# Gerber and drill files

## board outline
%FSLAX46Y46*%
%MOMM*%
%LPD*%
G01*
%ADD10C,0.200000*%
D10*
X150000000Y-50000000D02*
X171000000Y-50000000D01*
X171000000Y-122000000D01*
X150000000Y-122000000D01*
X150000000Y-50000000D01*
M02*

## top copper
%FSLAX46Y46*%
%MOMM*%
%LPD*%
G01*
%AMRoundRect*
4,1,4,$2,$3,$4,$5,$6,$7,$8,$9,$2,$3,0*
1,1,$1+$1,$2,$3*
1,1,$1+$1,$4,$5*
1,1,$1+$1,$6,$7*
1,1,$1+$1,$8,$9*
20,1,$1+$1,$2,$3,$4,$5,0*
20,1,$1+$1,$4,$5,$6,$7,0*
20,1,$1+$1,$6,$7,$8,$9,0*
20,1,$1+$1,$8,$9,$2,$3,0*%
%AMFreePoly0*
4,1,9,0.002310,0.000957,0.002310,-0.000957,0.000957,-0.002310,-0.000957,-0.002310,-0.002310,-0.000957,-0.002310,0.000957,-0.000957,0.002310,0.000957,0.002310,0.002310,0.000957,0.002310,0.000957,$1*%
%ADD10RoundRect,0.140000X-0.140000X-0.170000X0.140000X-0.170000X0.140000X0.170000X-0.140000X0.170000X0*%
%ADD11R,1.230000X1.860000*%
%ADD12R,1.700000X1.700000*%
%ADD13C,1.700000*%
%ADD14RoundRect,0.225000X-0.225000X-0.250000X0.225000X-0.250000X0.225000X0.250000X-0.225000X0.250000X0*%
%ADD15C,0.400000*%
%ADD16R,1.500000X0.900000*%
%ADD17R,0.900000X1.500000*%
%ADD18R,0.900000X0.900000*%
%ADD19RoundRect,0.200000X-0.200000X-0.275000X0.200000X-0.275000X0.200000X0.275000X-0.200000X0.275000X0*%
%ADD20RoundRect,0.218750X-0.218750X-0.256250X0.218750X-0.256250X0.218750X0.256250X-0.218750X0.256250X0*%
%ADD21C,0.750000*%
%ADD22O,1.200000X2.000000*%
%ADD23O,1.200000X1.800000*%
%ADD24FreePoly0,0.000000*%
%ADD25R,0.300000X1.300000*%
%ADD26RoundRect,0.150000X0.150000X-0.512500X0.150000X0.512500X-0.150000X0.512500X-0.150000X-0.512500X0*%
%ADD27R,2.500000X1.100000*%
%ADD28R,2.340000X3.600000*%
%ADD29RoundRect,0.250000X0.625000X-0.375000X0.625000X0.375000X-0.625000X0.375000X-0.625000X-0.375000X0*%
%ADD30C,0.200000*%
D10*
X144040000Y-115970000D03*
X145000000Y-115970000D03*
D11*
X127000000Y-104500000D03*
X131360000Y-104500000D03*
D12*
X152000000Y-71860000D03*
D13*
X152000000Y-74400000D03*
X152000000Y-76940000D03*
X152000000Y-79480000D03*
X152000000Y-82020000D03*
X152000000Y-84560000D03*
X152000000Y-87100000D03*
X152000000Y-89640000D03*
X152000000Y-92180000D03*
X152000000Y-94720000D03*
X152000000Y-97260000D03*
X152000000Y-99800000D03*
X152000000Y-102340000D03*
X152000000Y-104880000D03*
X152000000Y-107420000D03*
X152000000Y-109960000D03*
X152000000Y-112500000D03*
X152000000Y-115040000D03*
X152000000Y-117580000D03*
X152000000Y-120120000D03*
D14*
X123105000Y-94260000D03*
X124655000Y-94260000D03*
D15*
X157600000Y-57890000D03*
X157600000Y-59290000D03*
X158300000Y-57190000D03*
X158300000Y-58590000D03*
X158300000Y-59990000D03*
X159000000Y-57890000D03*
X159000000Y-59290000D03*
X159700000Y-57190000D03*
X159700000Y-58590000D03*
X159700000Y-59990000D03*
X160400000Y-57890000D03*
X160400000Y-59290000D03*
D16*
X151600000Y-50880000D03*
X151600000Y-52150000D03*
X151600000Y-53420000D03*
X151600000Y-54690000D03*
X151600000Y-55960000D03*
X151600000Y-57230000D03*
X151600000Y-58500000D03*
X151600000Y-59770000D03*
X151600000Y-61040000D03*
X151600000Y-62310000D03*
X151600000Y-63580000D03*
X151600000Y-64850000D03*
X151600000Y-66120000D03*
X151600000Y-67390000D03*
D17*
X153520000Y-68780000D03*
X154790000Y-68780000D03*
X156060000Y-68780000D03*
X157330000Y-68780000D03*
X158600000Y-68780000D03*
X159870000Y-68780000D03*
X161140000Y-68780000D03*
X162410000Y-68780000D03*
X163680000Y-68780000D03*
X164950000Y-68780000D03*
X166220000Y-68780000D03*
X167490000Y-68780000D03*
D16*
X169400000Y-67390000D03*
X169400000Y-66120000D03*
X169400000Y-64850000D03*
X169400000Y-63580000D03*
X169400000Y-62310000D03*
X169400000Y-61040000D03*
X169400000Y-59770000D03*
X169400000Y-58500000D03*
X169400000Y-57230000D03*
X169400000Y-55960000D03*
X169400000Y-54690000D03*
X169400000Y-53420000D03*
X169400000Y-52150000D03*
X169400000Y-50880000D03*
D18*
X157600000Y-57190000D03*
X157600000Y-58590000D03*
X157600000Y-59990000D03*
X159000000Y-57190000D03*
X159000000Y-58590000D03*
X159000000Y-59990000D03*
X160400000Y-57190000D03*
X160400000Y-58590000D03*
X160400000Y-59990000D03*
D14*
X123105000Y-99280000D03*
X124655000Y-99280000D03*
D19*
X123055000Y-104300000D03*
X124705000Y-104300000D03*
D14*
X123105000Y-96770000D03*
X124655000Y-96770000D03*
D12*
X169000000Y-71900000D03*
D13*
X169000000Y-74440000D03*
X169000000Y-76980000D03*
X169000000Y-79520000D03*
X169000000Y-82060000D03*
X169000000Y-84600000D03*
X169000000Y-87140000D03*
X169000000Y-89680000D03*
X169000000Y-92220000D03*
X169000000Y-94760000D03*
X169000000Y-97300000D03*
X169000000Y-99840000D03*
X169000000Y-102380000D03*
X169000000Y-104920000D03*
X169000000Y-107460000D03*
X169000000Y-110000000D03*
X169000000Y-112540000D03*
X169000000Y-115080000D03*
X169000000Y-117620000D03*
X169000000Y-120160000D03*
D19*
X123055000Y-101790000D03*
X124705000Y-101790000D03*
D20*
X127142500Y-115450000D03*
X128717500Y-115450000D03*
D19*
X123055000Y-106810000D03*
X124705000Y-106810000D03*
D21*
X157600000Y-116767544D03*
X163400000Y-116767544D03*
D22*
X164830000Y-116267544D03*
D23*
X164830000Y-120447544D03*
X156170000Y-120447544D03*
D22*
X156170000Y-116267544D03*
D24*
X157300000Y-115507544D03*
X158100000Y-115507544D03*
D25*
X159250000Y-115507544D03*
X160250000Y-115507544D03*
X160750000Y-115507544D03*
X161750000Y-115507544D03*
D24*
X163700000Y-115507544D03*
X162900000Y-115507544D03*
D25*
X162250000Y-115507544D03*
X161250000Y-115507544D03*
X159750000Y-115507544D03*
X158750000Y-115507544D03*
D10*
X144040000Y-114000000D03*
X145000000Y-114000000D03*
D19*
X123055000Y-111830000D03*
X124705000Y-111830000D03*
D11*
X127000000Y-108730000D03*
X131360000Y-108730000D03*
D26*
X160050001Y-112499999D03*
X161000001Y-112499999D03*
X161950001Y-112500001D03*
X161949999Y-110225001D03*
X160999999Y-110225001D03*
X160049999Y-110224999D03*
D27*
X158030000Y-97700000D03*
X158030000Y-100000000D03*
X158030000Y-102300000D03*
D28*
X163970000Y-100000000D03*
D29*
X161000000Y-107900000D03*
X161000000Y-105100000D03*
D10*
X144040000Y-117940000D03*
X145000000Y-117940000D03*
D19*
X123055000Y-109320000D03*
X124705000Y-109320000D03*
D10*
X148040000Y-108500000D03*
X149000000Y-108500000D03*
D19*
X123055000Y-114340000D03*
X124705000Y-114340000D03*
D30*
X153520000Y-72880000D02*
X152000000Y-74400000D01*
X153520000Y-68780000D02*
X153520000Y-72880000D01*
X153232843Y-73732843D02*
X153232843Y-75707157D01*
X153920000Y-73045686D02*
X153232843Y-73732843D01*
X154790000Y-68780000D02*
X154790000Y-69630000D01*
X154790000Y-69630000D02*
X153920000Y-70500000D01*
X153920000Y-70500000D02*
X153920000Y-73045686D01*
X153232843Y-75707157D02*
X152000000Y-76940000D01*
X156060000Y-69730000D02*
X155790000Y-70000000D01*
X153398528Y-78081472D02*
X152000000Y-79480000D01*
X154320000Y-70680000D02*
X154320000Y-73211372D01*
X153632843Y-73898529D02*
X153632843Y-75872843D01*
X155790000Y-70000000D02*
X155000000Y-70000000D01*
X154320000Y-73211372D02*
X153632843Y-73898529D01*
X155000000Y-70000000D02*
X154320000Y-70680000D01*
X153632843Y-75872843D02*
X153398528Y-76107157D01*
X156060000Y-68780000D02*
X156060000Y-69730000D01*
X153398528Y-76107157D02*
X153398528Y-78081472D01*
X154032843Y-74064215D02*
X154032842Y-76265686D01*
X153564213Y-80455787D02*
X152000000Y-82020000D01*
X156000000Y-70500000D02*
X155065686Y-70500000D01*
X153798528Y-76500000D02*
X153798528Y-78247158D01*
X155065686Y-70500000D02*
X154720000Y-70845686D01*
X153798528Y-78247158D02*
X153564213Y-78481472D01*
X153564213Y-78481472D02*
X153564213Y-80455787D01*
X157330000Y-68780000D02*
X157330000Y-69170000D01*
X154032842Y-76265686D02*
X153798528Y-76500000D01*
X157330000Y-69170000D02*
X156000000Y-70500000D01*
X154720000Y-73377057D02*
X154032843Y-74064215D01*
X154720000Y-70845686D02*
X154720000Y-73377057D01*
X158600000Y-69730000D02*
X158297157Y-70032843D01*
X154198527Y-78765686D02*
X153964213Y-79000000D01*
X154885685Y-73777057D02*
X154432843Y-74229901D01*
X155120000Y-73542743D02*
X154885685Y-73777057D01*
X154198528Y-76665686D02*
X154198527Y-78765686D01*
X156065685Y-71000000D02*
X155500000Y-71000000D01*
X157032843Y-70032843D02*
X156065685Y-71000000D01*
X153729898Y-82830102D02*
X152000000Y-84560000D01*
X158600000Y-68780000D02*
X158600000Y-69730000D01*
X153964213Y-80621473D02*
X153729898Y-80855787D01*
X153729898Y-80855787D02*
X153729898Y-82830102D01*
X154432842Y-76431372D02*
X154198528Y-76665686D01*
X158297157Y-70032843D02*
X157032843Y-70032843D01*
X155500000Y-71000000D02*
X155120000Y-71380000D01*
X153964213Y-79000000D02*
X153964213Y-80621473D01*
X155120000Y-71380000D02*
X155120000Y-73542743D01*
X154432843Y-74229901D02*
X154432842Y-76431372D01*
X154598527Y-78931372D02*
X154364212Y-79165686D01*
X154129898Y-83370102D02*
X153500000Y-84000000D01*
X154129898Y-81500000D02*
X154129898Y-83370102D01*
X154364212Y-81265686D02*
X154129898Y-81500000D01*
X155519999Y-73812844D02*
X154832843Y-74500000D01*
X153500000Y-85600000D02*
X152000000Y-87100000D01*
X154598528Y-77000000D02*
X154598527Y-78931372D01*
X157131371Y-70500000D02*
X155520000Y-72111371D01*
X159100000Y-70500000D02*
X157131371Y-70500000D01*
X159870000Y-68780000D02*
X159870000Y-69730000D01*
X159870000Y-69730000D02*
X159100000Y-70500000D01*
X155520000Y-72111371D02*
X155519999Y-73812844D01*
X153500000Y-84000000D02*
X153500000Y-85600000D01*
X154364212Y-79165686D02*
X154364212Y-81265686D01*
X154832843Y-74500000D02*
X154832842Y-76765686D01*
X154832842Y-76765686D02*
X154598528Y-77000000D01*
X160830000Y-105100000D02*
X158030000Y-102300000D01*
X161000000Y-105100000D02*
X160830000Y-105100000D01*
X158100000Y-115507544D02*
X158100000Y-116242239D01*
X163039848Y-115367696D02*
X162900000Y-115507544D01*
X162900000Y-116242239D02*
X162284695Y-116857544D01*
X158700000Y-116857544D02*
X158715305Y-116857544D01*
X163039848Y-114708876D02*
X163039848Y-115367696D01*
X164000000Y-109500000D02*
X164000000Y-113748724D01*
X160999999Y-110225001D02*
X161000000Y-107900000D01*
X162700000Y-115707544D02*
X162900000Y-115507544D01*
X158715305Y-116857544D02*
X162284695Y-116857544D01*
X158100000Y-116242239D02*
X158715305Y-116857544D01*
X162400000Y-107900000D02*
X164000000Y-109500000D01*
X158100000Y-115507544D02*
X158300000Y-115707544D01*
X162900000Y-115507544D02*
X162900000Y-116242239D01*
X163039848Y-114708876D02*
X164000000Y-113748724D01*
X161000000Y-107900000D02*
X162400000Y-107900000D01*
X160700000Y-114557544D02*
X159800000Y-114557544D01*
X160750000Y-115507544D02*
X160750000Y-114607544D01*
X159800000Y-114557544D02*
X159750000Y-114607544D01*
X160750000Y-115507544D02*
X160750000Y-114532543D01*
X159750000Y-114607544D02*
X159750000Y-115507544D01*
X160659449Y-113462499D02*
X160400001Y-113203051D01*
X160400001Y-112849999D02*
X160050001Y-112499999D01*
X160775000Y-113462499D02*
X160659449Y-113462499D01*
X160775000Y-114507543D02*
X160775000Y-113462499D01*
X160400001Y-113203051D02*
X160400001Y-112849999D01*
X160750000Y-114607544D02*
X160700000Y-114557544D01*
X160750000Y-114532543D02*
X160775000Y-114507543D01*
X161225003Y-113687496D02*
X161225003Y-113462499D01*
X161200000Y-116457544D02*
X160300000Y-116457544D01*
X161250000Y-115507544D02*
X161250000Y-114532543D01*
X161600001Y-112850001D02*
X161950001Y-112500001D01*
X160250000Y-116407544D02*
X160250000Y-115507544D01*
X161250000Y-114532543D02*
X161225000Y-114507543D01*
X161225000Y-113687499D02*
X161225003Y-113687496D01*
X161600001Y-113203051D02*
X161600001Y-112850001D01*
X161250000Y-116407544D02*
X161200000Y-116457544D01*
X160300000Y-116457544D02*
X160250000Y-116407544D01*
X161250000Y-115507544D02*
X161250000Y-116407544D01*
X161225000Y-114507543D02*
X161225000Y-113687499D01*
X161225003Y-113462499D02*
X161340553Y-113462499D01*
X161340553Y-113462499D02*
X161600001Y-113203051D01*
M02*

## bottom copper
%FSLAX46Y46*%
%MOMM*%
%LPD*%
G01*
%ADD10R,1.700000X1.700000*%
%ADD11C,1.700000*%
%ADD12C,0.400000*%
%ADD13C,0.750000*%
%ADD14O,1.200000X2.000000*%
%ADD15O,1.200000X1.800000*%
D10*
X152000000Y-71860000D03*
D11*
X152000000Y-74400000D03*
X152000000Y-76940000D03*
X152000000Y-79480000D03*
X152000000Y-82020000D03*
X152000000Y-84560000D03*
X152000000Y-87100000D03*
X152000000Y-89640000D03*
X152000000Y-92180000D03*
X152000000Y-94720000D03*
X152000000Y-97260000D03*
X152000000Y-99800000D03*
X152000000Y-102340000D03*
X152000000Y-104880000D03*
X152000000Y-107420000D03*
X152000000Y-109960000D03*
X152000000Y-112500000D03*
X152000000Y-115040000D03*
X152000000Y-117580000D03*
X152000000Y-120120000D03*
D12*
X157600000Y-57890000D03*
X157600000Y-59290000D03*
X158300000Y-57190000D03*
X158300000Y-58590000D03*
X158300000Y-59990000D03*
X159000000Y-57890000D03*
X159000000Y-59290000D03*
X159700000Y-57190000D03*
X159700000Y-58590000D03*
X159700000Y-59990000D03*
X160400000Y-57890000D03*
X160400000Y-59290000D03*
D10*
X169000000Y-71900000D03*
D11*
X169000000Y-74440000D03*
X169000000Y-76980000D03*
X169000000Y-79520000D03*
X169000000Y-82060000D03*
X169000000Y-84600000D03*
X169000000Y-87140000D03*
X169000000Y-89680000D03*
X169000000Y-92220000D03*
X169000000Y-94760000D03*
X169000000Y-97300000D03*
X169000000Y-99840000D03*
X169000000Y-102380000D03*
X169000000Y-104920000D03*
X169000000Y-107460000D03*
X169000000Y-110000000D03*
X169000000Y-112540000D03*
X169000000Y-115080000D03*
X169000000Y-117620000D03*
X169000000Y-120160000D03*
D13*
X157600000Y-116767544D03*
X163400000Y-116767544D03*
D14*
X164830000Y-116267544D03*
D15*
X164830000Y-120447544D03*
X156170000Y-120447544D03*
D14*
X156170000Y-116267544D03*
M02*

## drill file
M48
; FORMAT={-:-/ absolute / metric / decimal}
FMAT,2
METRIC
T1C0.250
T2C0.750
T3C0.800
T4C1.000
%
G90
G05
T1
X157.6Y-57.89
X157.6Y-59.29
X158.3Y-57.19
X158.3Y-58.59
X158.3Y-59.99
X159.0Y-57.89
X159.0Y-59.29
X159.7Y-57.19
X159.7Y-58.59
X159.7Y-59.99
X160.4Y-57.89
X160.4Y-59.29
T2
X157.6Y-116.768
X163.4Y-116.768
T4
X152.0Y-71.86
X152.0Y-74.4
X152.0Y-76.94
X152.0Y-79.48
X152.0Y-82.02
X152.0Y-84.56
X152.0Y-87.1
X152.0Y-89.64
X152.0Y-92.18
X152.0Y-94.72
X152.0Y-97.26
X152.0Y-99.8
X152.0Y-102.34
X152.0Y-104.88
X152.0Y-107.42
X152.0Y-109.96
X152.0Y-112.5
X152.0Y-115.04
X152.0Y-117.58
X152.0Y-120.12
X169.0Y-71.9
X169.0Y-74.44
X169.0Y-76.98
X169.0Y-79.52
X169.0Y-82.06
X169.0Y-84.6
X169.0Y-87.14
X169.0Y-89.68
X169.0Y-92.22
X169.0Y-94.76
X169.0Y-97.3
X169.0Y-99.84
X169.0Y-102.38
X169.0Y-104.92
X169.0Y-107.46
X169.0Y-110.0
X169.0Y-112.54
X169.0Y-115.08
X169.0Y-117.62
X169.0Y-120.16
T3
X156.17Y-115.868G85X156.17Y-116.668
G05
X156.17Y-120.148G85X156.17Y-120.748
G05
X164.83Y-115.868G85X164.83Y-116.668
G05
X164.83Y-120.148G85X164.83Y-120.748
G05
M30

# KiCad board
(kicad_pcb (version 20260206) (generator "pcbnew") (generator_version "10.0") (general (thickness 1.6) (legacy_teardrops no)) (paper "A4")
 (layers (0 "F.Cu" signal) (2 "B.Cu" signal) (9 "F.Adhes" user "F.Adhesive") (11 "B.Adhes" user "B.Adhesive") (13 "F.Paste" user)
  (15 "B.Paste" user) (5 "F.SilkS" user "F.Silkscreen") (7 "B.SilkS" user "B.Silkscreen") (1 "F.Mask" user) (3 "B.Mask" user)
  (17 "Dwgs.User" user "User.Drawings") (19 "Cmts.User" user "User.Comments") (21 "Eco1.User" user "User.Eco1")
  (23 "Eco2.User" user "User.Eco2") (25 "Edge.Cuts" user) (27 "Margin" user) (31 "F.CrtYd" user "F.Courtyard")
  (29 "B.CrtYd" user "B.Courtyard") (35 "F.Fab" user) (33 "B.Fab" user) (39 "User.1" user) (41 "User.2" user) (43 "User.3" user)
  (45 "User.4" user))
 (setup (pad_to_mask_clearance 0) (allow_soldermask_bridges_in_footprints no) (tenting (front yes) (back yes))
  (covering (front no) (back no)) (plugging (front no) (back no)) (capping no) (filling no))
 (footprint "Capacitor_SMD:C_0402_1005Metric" (layer "F.Cu") (at 144.52 115.97)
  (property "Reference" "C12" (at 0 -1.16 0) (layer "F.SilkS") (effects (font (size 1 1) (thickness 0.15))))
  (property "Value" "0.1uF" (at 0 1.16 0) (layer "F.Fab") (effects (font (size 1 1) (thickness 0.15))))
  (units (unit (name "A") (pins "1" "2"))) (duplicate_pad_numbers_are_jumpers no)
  (pad "1" smd roundrect (at -0.48 0) (size 0.56 0.62) (layers "F.Cu" "F.Mask" "F.Paste") (roundrect_rratio 0.25) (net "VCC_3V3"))
  (pad "2" smd roundrect (at 0.48 0) (size 0.56 0.62) (layers "F.Cu" "F.Mask" "F.Paste") (roundrect_rratio 0.25) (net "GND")))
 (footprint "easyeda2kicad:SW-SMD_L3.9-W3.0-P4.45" (layer "F.Cu") (at 129.18 104.5)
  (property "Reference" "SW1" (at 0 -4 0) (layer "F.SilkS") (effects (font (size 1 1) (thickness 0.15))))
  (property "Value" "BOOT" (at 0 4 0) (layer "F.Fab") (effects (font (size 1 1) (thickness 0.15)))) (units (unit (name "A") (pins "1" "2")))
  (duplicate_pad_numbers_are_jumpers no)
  (pad "1" smd rect (at -2.18 0) (size 1.23 1.86) (layers "F.Cu" "F.Mask" "F.Paste") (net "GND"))
  (pad "2" smd rect (at 2.18 0) (size 1.23 1.86) (layers "F.Cu" "F.Mask" "F.Paste") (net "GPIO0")))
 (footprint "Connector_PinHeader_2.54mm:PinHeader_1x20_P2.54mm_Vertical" (layer "F.Cu") (at 152 71.86)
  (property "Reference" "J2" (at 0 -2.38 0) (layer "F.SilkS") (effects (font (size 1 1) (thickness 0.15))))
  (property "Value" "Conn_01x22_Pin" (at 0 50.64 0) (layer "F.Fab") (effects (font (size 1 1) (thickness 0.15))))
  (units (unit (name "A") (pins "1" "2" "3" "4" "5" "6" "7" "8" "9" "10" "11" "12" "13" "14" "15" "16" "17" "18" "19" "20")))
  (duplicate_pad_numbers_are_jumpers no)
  (pad "1" thru_hole rect (at 0 0) (size 1.7 1.7) (drill 1) (layers "*.Cu" "*.Mask") (remove_unused_layers no) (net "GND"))
  (pad "2" thru_hole circle (at 0 2.54) (size 1.7 1.7) (drill 1) (layers "*.Cu" "*.Mask") (remove_unused_layers no) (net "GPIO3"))
  (pad "3" thru_hole circle (at 0 5.08) (size 1.7 1.7) (drill 1) (layers "*.Cu" "*.Mask") (remove_unused_layers no) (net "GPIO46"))
  (pad "4" thru_hole circle (at 0 7.62) (size 1.7 1.7) (drill 1) (layers "*.Cu" "*.Mask") (remove_unused_layers no) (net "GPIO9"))
  (pad "5" thru_hole circle (at 0 10.16) (size 1.7 1.7) (drill 1) (layers "*.Cu" "*.Mask") (remove_unused_layers no) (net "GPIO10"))
  (pad "6" thru_hole circle (at 0 12.7) (size 1.7 1.7) (drill 1) (layers "*.Cu" "*.Mask") (remove_unused_layers no) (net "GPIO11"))
  (pad "7" thru_hole circle (at 0 15.24) (size 1.7 1.7) (drill 1) (layers "*.Cu" "*.Mask") (remove_unused_layers no) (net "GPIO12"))
  (pad "8" thru_hole circle (at 0 17.78) (size 1.7 1.7) (drill 1) (layers "*.Cu" "*.Mask") (remove_unused_layers no) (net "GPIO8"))
  (pad "9" thru_hole circle (at 0 20.32) (size 1.7 1.7) (drill 1) (layers "*.Cu" "*.Mask") (remove_unused_layers no) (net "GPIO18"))
  (pad "10" thru_hole circle (at 0 22.86) (size 1.7 1.7) (drill 1) (layers "*.Cu" "*.Mask") (remove_unused_layers no) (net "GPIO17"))
  (pad "11" thru_hole circle (at 0 25.4) (size 1.7 1.7) (drill 1) (layers "*.Cu" "*.Mask") (remove_unused_layers no) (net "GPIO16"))
  (pad "12" thru_hole circle (at 0 27.94) (size 1.7 1.7) (drill 1) (layers "*.Cu" "*.Mask") (remove_unused_layers no) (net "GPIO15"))
  (pad "13" thru_hole circle (at 0 30.48) (size 1.7 1.7) (drill 1) (layers "*.Cu" "*.Mask") (remove_unused_layers no) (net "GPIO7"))
  (pad "14" thru_hole circle (at 0 33.02) (size 1.7 1.7) (drill 1) (layers "*.Cu" "*.Mask") (remove_unused_layers no) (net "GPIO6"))
  (pad "15" thru_hole circle (at 0 35.56) (size 1.7 1.7) (drill 1) (layers "*.Cu" "*.Mask") (remove_unused_layers no) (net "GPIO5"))
  (pad "16" thru_hole circle (at 0 38.1) (size 1.7 1.7) (drill 1) (layers "*.Cu" "*.Mask") (remove_unused_layers no) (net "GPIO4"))
  (pad "17" thru_hole circle (at 0 40.64) (size 1.7 1.7) (drill 1) (layers "*.Cu" "*.Mask") (remove_unused_layers no) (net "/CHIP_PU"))
  (pad "18" thru_hole circle (at 0 43.18) (size 1.7 1.7) (drill 1) (layers "*.Cu" "*.Mask") (remove_unused_layers no) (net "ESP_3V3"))
  (pad "19" thru_hole circle (at 0 45.72) (size 1.7 1.7) (drill 1) (layers "*.Cu" "*.Mask") (remove_unused_layers no) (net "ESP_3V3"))
  (pad "20" thru_hole circle (at 0 48.26) (size 1.7 1.7) (drill 1) (layers "*.Cu" "*.Mask") (remove_unused_layers no) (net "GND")))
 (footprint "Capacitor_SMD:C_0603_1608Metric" (layer "F.Cu") (at 123.88 94.26)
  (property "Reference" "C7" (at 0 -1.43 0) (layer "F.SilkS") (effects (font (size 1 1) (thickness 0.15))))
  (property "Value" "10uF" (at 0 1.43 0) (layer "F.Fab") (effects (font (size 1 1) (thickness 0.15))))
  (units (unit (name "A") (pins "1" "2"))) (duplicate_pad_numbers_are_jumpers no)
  (pad "1" smd roundrect (at -0.775 0) (size 0.9 0.95) (layers "F.Cu" "F.Mask" "F.Paste") (roundrect_rratio 0.25) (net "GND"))
  (pad "2" smd roundrect (at 0.775 0) (size 0.9 0.95) (layers "F.Cu" "F.Mask" "F.Paste") (roundrect_rratio 0.25) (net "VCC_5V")))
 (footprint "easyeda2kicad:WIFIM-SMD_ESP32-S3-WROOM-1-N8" (layer "F.Cu") (at 160.5 59.83)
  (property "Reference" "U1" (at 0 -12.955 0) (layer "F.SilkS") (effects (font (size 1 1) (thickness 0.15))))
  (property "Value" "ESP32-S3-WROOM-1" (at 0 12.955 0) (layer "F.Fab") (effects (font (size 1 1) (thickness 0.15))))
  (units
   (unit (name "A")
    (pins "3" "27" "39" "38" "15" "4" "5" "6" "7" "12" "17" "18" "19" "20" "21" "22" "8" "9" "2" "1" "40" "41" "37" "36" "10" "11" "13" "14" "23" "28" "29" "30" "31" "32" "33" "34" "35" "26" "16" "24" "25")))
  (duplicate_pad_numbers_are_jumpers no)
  (pad "" thru_hole circle (at -2.9 -1.94) (size 0.4 0.4) (drill 0.25) (layers "*.Cu" "*.Paste" "*.Mask") (remove_unused_layers no))
  (pad "" thru_hole circle (at -2.9 -0.54) (size 0.4 0.4) (drill 0.25) (layers "*.Cu" "*.Paste" "*.Mask") (remove_unused_layers no))
  (pad "" thru_hole circle (at -2.2 -2.64) (size 0.4 0.4) (drill 0.25) (layers "*.Cu" "*.Paste" "*.Mask") (remove_unused_layers no))
  (pad "" thru_hole circle (at -2.2 -1.24) (size 0.4 0.4) (drill 0.25) (layers "*.Cu" "*.Paste" "*.Mask") (remove_unused_layers no))
  (pad "" thru_hole circle (at -2.2 0.16) (size 0.4 0.4) (drill 0.25) (layers "*.Cu" "*.Paste" "*.Mask") (remove_unused_layers no))
  (pad "" thru_hole circle (at -1.5 -1.94) (size 0.4 0.4) (drill 0.25) (layers "*.Cu" "*.Paste" "*.Mask") (remove_unused_layers no))
  (pad "" thru_hole circle (at -1.5 -0.54) (size 0.4 0.4) (drill 0.25) (layers "*.Cu" "*.Paste" "*.Mask") (remove_unused_layers no))
  (pad "" thru_hole circle (at -0.8 -2.64) (size 0.4 0.4) (drill 0.25) (layers "*.Cu" "*.Paste" "*.Mask") (remove_unused_layers no))
  (pad "" thru_hole circle (at -0.8 -1.24) (size 0.4 0.4) (drill 0.25) (layers "*.Cu" "*.Paste" "*.Mask") (remove_unused_layers no))
  (pad "" thru_hole circle (at -0.8 0.16) (size 0.4 0.4) (drill 0.25) (layers "*.Cu" "*.Paste" "*.Mask") (remove_unused_layers no))
  (pad "" thru_hole circle (at -0.1 -1.94) (size 0.4 0.4) (drill 0.25) (layers "*.Cu" "*.Paste" "*.Mask") (remove_unused_layers no))
  (pad "" thru_hole circle (at -0.1 -0.54) (size 0.4 0.4) (drill 0.25) (layers "*.Cu" "*.Paste" "*.Mask") (remove_unused_layers no))
  (pad "1" smd rect (at -8.9 -8.95) (size 1.5 0.9) (layers "F.Cu" "F.Mask" "F.Paste") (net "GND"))
  (pad "2" smd rect (at -8.9 -7.68) (size 1.5 0.9) (layers "F.Cu" "F.Mask" "F.Paste") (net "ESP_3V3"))
  (pad "3" smd rect (at -8.9 -6.41) (size 1.5 0.9) (layers "F.Cu" "F.Mask" "F.Paste") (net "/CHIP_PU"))
  (pad "4" smd rect (at -8.9 -5.14) (size 1.5 0.9) (layers "F.Cu" "F.Mask" "F.Paste") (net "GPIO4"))
  (pad "5" smd rect (at -8.9 -3.87) (size 1.5 0.9) (layers "F.Cu" "F.Mask" "F.Paste") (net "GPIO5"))
  (pad "6" smd rect (at -8.9 -2.6) (size 1.5 0.9) (layers "F.Cu" "F.Mask" "F.Paste") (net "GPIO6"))
  (pad "7" smd rect (at -8.9 -1.33) (size 1.5 0.9) (layers "F.Cu" "F.Mask" "F.Paste") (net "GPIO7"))
  (pad "8" smd rect (at -8.9 -0.06) (size 1.5 0.9) (layers "F.Cu" "F.Mask" "F.Paste") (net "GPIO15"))
  (pad "9" smd rect (at -8.9 1.21) (size 1.5 0.9) (layers "F.Cu" "F.Mask" "F.Paste") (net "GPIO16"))
  (pad "10" smd rect (at -8.9 2.48) (size 1.5 0.9) (layers "F.Cu" "F.Mask" "F.Paste") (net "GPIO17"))
  (pad "11" smd rect (at -8.9 3.75) (size 1.5 0.9) (layers "F.Cu" "F.Mask" "F.Paste") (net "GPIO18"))
  (pad "12" smd rect (at -8.9 5.02) (size 1.5 0.9) (layers "F.Cu" "F.Mask" "F.Paste") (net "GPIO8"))
  (pad "13" smd rect (at -8.9 6.29) (size 1.5 0.9) (layers "F.Cu" "F.Mask" "F.Paste") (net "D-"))
  (pad "14" smd rect (at -8.9 7.56) (size 1.5 0.9) (layers "F.Cu" "F.Mask" "F.Paste") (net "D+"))
  (pad "15" smd rect (at -6.98 8.95) (size 0.9 1.5) (layers "F.Cu" "F.Mask" "F.Paste") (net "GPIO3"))
  (pad "16" smd rect (at -5.71 8.95) (size 0.9 1.5) (layers "F.Cu" "F.Mask" "F.Paste") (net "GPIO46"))
  (pad "17" smd rect (at -4.44 8.95) (size 0.9 1.5) (layers "F.Cu" "F.Mask" "F.Paste") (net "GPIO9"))
  (pad "18" smd rect (at -3.17 8.95) (size 0.9 1.5) (layers "F.Cu" "F.Mask" "F.Paste") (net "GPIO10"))
  (pad "19" smd rect (at -1.9 8.95) (size 0.9 1.5) (layers "F.Cu" "F.Mask" "F.Paste") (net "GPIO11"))
  (pad "20" smd rect (at -0.63 8.95) (size 0.9 1.5) (layers "F.Cu" "F.Mask" "F.Paste") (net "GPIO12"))
  (pad "21" smd rect (at 0.64 8.95) (size 0.9 1.5) (layers "F.Cu" "F.Mask" "F.Paste") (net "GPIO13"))
  (pad "22" smd rect (at 1.91 8.95) (size 0.9 1.5) (layers "F.Cu" "F.Mask" "F.Paste") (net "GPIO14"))
  (pad "23" smd rect (at 3.18 8.95) (size 0.9 1.5) (layers "F.Cu" "F.Mask" "F.Paste") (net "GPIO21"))
  (pad "24" smd rect (at 4.45 8.95) (size 0.9 1.5) (layers "F.Cu" "F.Mask" "F.Paste") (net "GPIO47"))
  (pad "25" smd rect (at 5.72 8.95) (size 0.9 1.5) (layers "F.Cu" "F.Mask" "F.Paste") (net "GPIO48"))
  (pad "26" smd rect (at 6.99 8.95) (size 0.9 1.5) (layers "F.Cu" "F.Mask" "F.Paste") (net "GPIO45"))
  (pad "27" smd rect (at 8.9 7.56) (size 1.5 0.9) (layers "F.Cu" "F.Mask" "F.Paste") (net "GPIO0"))
  (pad "28" smd rect (at 8.9 6.29) (size 1.5 0.9) (layers "F.Cu" "F.Mask" "F.Paste") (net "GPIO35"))
  (pad "29" smd rect (at 8.9 5.02) (size 1.5 0.9) (layers "F.Cu" "F.Mask" "F.Paste") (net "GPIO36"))
  (pad "30" smd rect (at 8.9 3.75) (size 1.5 0.9) (layers "F.Cu" "F.Mask" "F.Paste") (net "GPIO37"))
  (pad "31" smd rect (at 8.9 2.48) (size 1.5 0.9) (layers "F.Cu" "F.Mask" "F.Paste") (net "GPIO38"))
  (pad "32" smd rect (at 8.9 1.21) (size 1.5 0.9) (layers "F.Cu" "F.Mask" "F.Paste") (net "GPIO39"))
  (pad "33" smd rect (at 8.9 -0.06) (size 1.5 0.9) (layers "F.Cu" "F.Mask" "F.Paste") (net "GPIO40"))
  (pad "34" smd rect (at 8.9 -1.33) (size 1.5 0.9) (layers "F.Cu" "F.Mask" "F.Paste") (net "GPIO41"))
  (pad "35" smd rect (at 8.9 -2.6) (size 1.5 0.9) (layers "F.Cu" "F.Mask" "F.Paste") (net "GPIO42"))
  (pad "36" smd rect (at 8.9 -3.87) (size 1.5 0.9) (layers "F.Cu" "F.Mask" "F.Paste") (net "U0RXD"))
  (pad "37" smd rect (at 8.9 -5.14) (size 1.5 0.9) (layers "F.Cu" "F.Mask" "F.Paste") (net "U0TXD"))
  (pad "38" smd rect (at 8.9 -6.41) (size 1.5 0.9) (layers "F.Cu" "F.Mask" "F.Paste") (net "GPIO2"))
  (pad "39" smd rect (at 8.9 -7.68) (size 1.5 0.9) (layers "F.Cu" "F.Mask" "F.Paste") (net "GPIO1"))
  (pad "40" smd rect (at 8.9 -8.95) (size 1.5 0.9) (layers "F.Cu" "F.Mask" "F.Paste") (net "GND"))
  (pad "41" smd rect (at -2.9 -2.64 90) (size 0.9 0.9) (layers "F.Cu" "F.Mask" "F.Paste") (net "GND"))
  (pad "41" smd rect (at -2.9 -1.24 90) (size 0.9 0.9) (layers "F.Cu" "F.Mask" "F.Paste") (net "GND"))
  (pad "41" smd rect (at -2.9 0.16 90) (size 0.9 0.9) (layers "F.Cu" "F.Mask" "F.Paste") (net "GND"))
  (pad "41" smd rect (at -1.5 -2.64 90) (size 0.9 0.9) (layers "F.Cu" "F.Mask" "F.Paste") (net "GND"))
  (pad "41" smd rect (at -1.5 -1.24 90) (size 0.9 0.9) (layers "F.Cu" "F.Mask" "F.Paste") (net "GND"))
  (pad "41" smd rect (at -1.5 0.16 90) (size 0.9 0.9) (layers "F.Cu" "F.Mask" "F.Paste") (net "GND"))
  (pad "41" smd rect (at -0.1 -2.64 90) (size 0.9 0.9) (layers "F.Cu" "F.Mask" "F.Paste") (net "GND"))
  (pad "41" smd rect (at -0.1 -1.24 90) (size 0.9 0.9) (layers "F.Cu" "F.Mask" "F.Paste") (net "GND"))
  (pad "41" smd rect (at -0.1 0.16 90) (size 0.9 0.9) (layers "F.Cu" "F.Mask" "F.Paste") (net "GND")))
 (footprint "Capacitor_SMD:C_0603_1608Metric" (layer "F.Cu") (at 123.88 99.28)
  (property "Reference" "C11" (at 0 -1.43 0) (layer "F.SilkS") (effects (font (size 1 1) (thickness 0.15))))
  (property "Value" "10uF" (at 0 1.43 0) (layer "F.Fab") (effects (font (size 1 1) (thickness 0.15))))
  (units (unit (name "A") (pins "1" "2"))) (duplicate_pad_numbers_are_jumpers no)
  (pad "1" smd roundrect (at -0.775 0) (size 0.9 0.95) (layers "F.Cu" "F.Mask" "F.Paste") (roundrect_rratio 0.25) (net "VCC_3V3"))
  (pad "2" smd roundrect (at 0.775 0) (size 0.9 0.95) (layers "F.Cu" "F.Mask" "F.Paste") (roundrect_rratio 0.25) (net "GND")))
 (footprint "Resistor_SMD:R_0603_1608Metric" (layer "F.Cu") (at 123.88 104.3)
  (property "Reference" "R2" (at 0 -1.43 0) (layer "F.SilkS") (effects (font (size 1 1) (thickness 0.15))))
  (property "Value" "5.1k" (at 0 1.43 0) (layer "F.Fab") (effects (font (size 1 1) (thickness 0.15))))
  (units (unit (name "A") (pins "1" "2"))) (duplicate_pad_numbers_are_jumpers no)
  (pad "1" smd roundrect (at -0.825 0) (size 0.8 0.95) (layers "F.Cu" "F.Mask" "F.Paste") (roundrect_rratio 0.25) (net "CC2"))
  (pad "2" smd roundrect (at 0.825 0) (size 0.8 0.95) (layers "F.Cu" "F.Mask" "F.Paste") (roundrect_rratio 0.25) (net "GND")))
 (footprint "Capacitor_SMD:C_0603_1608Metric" (layer "F.Cu") (at 123.88 96.77)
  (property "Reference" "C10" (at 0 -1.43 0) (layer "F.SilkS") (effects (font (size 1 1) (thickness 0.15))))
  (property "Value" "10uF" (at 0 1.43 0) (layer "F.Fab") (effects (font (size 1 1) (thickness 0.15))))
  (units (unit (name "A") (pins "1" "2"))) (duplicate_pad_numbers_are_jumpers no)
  (pad "1" smd roundrect (at -0.775 0) (size 0.9 0.95) (layers "F.Cu" "F.Mask" "F.Paste") (roundrect_rratio 0.25) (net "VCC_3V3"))
  (pad "2" smd roundrect (at 0.775 0) (size 0.9 0.95) (layers "F.Cu" "F.Mask" "F.Paste") (roundrect_rratio 0.25) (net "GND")))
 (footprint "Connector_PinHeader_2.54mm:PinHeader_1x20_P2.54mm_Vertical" (layer "F.Cu") (at 169 71.9)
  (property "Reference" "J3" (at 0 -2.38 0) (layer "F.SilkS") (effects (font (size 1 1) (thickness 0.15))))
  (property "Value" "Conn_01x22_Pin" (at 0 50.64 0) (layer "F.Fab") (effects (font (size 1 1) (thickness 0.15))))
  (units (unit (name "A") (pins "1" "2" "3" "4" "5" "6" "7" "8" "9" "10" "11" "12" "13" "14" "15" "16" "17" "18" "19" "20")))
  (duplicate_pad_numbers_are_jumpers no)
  (pad "1" thru_hole rect (at 0 0) (size 1.7 1.7) (drill 1) (layers "*.Cu" "*.Mask") (remove_unused_layers no) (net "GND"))
  (pad "2" thru_hole circle (at 0 2.54) (size 1.7 1.7) (drill 1) (layers "*.Cu" "*.Mask") (remove_unused_layers no) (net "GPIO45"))
  (pad "3" thru_hole circle (at 0 5.08) (size 1.7 1.7) (drill 1) (layers "*.Cu" "*.Mask") (remove_unused_layers no) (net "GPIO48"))
  (pad "4" thru_hole circle (at 0 7.62) (size 1.7 1.7) (drill 1) (layers "*.Cu" "*.Mask") (remove_unused_layers no) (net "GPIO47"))
  (pad "5" thru_hole circle (at 0 10.16) (size 1.7 1.7) (drill 1) (layers "*.Cu" "*.Mask") (remove_unused_layers no) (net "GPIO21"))
  (pad "6" thru_hole circle (at 0 12.7) (size 1.7 1.7) (drill 1) (layers "*.Cu" "*.Mask") (remove_unused_layers no) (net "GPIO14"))
  (pad "7" thru_hole circle (at 0 15.24) (size 1.7 1.7) (drill 1) (layers "*.Cu" "*.Mask") (remove_unused_layers no) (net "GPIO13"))
  (pad "8" thru_hole circle (at 0 17.78) (size 1.7 1.7) (drill 1) (layers "*.Cu" "*.Mask") (remove_unused_layers no) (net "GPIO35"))
  (pad "9" thru_hole circle (at 0 20.32) (size 1.7 1.7) (drill 1) (layers "*.Cu" "*.Mask") (remove_unused_layers no) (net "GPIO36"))
  (pad "10" thru_hole circle (at 0 22.86) (size 1.7 1.7) (drill 1) (layers "*.Cu" "*.Mask") (remove_unused_layers no) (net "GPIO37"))
  (pad "11" thru_hole circle (at 0 25.4) (size 1.7 1.7) (drill 1) (layers "*.Cu" "*.Mask") (remove_unused_layers no) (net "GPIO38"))
  (pad "12" thru_hole circle (at 0 27.94) (size 1.7 1.7) (drill 1) (layers "*.Cu" "*.Mask") (remove_unused_layers no) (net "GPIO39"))
  (pad "13" thru_hole circle (at 0 30.48) (size 1.7 1.7) (drill 1) (layers "*.Cu" "*.Mask") (remove_unused_layers no) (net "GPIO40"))
  (pad "14" thru_hole circle (at 0 33.02) (size 1.7 1.7) (drill 1) (layers "*.Cu" "*.Mask") (remove_unused_layers no) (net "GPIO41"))
  (pad "15" thru_hole circle (at 0 35.56) (size 1.7 1.7) (drill 1) (layers "*.Cu" "*.Mask") (remove_unused_layers no) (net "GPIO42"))
  (pad "16" thru_hole circle (at 0 38.1) (size 1.7 1.7) (drill 1) (layers "*.Cu" "*.Mask") (remove_unused_layers no) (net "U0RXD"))
  (pad "17" thru_hole circle (at 0 40.64) (size 1.7 1.7) (drill 1) (layers "*.Cu" "*.Mask") (remove_unused_layers no) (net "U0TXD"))
  (pad "18" thru_hole circle (at 0 43.18) (size 1.7 1.7) (drill 1) (layers "*.Cu" "*.Mask") (remove_unused_layers no) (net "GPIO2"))
  (pad "19" thru_hole circle (at 0 45.72) (size 1.7 1.7) (drill 1) (layers "*.Cu" "*.Mask") (remove_unused_layers no) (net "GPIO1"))
  (pad "20" thru_hole circle (at 0 48.26) (size 1.7 1.7) (drill 1) (layers "*.Cu" "*.Mask") (remove_unused_layers no) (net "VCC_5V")))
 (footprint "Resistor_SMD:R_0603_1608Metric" (layer "F.Cu") (at 123.88 101.79)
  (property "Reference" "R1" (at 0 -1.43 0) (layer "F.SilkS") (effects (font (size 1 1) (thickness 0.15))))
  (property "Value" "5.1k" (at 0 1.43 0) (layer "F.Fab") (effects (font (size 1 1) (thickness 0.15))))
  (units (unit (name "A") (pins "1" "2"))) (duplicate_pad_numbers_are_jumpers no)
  (pad "1" smd roundrect (at -0.825 0) (size 0.8 0.95) (layers "F.Cu" "F.Mask" "F.Paste") (roundrect_rratio 0.25) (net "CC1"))
  (pad "2" smd roundrect (at 0.825 0) (size 0.8 0.95) (layers "F.Cu" "F.Mask" "F.Paste") (roundrect_rratio 0.25) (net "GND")))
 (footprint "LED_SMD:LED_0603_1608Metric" (layer "F.Cu") (at 127.93 115.45)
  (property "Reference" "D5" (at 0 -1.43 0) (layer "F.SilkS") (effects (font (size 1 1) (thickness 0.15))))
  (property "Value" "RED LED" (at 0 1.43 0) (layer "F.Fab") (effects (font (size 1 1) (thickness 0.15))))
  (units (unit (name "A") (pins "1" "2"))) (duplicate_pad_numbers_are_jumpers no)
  (pad "1" smd roundrect (at -0.7875 0) (size 0.875 0.95) (layers "F.Cu" "F.Mask" "F.Paste") (roundrect_rratio 0.25) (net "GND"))
  (pad "2" smd roundrect (at 0.7875 0) (size 0.875 0.95) (layers "F.Cu" "F.Mask" "F.Paste") (roundrect_rratio 0.25) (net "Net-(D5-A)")))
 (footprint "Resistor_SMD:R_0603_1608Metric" (layer "F.Cu") (at 123.88 106.81)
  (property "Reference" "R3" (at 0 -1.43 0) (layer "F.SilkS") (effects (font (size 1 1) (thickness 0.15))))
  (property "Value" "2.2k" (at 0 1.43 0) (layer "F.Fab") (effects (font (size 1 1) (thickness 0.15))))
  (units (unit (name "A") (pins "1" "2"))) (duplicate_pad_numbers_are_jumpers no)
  (pad "1" smd roundrect (at -0.825 0) (size 0.8 0.95) (layers "F.Cu" "F.Mask" "F.Paste") (roundrect_rratio 0.25) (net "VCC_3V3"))
  (pad "2" smd roundrect (at 0.825 0) (size 0.8 0.95) (layers "F.Cu" "F.Mask" "F.Paste") (roundrect_rratio 0.25) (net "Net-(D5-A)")))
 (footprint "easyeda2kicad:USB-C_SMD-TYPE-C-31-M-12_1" (layer "F.Cu") (at 160.5 117.977544)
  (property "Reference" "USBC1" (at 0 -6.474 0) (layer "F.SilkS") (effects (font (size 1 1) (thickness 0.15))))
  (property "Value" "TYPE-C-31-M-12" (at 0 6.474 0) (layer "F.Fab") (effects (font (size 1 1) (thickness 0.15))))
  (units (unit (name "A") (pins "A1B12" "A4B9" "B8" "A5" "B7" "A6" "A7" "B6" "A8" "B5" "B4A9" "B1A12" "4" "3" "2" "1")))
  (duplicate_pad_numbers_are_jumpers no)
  (pad "" thru_hole circle (at -2.9 -1.21) (size 0.75 0.75) (drill 0.75) (layers "*.Cu" "*.Mask") (remove_unused_layers no))
  (pad "" thru_hole circle (at 2.9 -1.21) (size 0.75 0.75) (drill 0.75) (layers "*.Cu" "*.Mask") (remove_unused_layers no))
  (pad "1" thru_hole oval (at 4.33 -1.71) (size 1.2 2) (drill oval 0.799998 1.599971) (layers "*.Cu" "*.Mask") (remove_unused_layers no)
   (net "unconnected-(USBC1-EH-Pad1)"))
  (pad "2" thru_hole oval (at 4.33 2.47) (size 1.2 1.8) (drill oval 0.799998 1.399997) (layers "*.Cu" "*.Mask") (remove_unused_layers no)
   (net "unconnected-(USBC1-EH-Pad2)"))
  (pad "3" thru_hole oval (at -4.33 2.47) (size 1.2 1.8) (drill oval 0.799998 1.399997) (layers "*.Cu" "*.Mask") (remove_unused_layers no)
   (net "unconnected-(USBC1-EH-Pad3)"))
  (pad "4" thru_hole oval (at -4.33 -1.71) (size 1.2 2) (drill oval 0.799998 1.600022) (layers "*.Cu" "*.Mask") (remove_unused_layers no)
   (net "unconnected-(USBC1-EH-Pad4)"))
  (pad "A1B12" smd custom (at -3.2 -2.47) (size 0.005 0.005) (layers "F.Cu" "F.Mask" "F.Paste") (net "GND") (thermal_bridge_angle 90)
   (options (clearance outline) (anchor circle)) (primitives))
  (pad "A4B9" smd custom (at -2.4 -2.47) (size 0.005 0.005) (layers "F.Cu" "F.Mask" "F.Paste") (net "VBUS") (thermal_bridge_angle 90)
   (options (clearance outline) (anchor circle)) (primitives))
  (pad "A5" smd rect (at -1.25 -2.47) (size 0.3 1.3) (layers "F.Cu" "F.Mask" "F.Paste") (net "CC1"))
  (pad "A6" smd rect (at -0.25 -2.47) (size 0.3 1.3) (layers "F.Cu" "F.Mask" "F.Paste") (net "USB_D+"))
  (pad "A7" smd rect (at 0.25 -2.47) (size 0.3 1.3) (layers "F.Cu" "F.Mask" "F.Paste") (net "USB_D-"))
  (pad "A8" smd rect (at 1.25 -2.47) (size 0.3 1.3) (layers "F.Cu" "F.Mask" "F.Paste") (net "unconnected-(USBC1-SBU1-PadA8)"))
  (pad "B1A12" smd custom (at 3.2 -2.47) (size 0.005 0.005) (layers "F.Cu" "F.Mask" "F.Paste") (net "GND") (thermal_bridge_angle 90)
   (options (clearance outline) (anchor circle)) (primitives))
  (pad "B4A9" smd custom (at 2.4 -2.47) (size 0.005 0.005) (layers "F.Cu" "F.Mask" "F.Paste") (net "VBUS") (thermal_bridge_angle 90)
   (options (clearance outline) (anchor circle)) (primitives))
  (pad "B5" smd rect (at 1.75 -2.47) (size 0.3 1.3) (layers "F.Cu" "F.Mask" "F.Paste") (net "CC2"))
  (pad "B6" smd rect (at 0.75 -2.47) (size 0.3 1.3) (layers "F.Cu" "F.Mask" "F.Paste") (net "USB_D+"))
  (pad "B7" smd rect (at -0.75 -2.47) (size 0.3 1.3) (layers "F.Cu" "F.Mask" "F.Paste") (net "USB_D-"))
  (pad "B8" smd rect (at -1.75 -2.47) (size 0.3 1.3) (layers "F.Cu" "F.Mask" "F.Paste") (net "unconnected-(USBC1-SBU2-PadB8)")))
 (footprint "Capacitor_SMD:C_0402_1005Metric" (layer "F.Cu") (at 144.52 114)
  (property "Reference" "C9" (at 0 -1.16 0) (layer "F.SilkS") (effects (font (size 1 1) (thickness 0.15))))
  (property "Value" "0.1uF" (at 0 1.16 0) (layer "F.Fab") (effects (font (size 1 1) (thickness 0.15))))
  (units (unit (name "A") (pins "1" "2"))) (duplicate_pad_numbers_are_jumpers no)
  (pad "1" smd roundrect (at -0.48 0) (size 0.56 0.62) (layers "F.Cu" "F.Mask" "F.Paste") (roundrect_rratio 0.25) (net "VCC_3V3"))
  (pad "2" smd roundrect (at 0.48 0) (size 0.56 0.62) (layers "F.Cu" "F.Mask" "F.Paste") (roundrect_rratio 0.25) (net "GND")))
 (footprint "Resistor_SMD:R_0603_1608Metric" (layer "F.Cu") (at 123.88 111.83)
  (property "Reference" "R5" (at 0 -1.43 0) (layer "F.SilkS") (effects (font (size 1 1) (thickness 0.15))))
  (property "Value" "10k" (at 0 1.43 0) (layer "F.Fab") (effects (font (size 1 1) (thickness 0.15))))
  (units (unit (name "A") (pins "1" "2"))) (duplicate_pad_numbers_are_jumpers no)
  (pad "1" smd roundrect (at -0.825 0) (size 0.8 0.95) (layers "F.Cu" "F.Mask" "F.Paste") (roundrect_rratio 0.25) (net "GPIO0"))
  (pad "2" smd roundrect (at 0.825 0) (size 0.8 0.95) (layers "F.Cu" "F.Mask" "F.Paste") (roundrect_rratio 0.25) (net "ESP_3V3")))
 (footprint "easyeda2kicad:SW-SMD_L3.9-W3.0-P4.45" (layer "F.Cu") (at 129.18 108.73)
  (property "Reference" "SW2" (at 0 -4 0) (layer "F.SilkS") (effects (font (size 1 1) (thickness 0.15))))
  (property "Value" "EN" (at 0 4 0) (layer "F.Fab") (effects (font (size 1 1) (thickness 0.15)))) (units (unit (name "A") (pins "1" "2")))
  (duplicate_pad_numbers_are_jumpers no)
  (pad "1" smd rect (at -2.18 0) (size 1.23 1.86) (layers "F.Cu" "F.Mask" "F.Paste") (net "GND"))
  (pad "2" smd rect (at 2.18 0) (size 1.23 1.86) (layers "F.Cu" "F.Mask" "F.Paste") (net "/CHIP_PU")))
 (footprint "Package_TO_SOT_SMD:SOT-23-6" (layer "F.Cu") (at 161 111.3625 90)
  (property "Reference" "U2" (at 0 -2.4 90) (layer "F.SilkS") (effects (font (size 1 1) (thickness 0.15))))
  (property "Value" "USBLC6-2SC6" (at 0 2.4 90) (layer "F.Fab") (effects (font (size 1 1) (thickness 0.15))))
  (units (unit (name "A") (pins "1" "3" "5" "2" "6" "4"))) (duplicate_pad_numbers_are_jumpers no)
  (pad "1" smd roundrect (at -1.137499 -0.949999 90) (size 1.325 0.6) (layers "F.Cu" "F.Mask" "F.Paste") (roundrect_rratio 0.25)
   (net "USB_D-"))
  (pad "2" smd roundrect (at -1.137499 0.000001 90) (size 1.325 0.6) (layers "F.Cu" "F.Mask" "F.Paste") (roundrect_rratio 0.25) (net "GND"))
  (pad "3" smd roundrect (at -1.137501 0.950001 90) (size 1.325 0.6) (layers "F.Cu" "F.Mask" "F.Paste") (roundrect_rratio 0.25)
   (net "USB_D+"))
  (pad "4" smd roundrect (at 1.137499 0.949999 90) (size 1.325 0.6) (layers "F.Cu" "F.Mask" "F.Paste") (roundrect_rratio 0.25) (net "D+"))
  (pad "5" smd roundrect (at 1.137499 -0.000001 90) (size 1.325 0.6) (layers "F.Cu" "F.Mask" "F.Paste") (roundrect_rratio 0.25) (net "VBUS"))
  (pad "6" smd roundrect (at 1.137501 -0.950001 90) (size 1.325 0.6) (layers "F.Cu" "F.Mask" "F.Paste") (roundrect_rratio 0.25) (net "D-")))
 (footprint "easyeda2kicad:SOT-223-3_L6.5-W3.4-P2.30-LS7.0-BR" (layer "F.Cu") (at 161 100 180)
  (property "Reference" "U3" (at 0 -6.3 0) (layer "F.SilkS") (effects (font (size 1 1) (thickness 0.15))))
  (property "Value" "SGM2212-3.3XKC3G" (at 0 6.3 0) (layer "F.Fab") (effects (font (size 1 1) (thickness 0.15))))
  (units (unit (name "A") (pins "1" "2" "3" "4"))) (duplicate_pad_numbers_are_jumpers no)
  (pad "1" smd rect (at 2.97 2.3 180) (size 2.5 1.1) (layers "F.Cu" "F.Mask" "F.Paste") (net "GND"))
  (pad "2" smd rect (at 2.97 0 180) (size 2.5 1.1) (layers "F.Cu" "F.Mask" "F.Paste") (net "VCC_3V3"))
  (pad "3" smd rect (at 2.97 -2.3 180) (size 2.5 1.1) (layers "F.Cu" "F.Mask" "F.Paste") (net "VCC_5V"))
  (pad "4" smd rect (at -2.97 0 180) (size 2.34 3.6) (layers "F.Cu" "F.Mask" "F.Paste") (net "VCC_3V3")))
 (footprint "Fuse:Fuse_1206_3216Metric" (layer "F.Cu") (at 161 106.5 90)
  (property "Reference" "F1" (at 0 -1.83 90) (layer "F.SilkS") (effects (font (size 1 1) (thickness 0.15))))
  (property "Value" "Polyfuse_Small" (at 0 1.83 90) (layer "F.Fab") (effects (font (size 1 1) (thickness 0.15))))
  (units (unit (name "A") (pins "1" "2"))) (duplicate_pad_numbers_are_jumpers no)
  (pad "1" smd roundrect (at -1.4 0 90) (size 1.25 1.75) (layers "F.Cu" "F.Mask" "F.Paste") (roundrect_rratio 0.2) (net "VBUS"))
  (pad "2" smd roundrect (at 1.4 0 90) (size 1.25 1.75) (layers "F.Cu" "F.Mask" "F.Paste") (roundrect_rratio 0.2) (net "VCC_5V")))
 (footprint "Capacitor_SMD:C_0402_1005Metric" (layer "F.Cu") (at 144.52 117.94)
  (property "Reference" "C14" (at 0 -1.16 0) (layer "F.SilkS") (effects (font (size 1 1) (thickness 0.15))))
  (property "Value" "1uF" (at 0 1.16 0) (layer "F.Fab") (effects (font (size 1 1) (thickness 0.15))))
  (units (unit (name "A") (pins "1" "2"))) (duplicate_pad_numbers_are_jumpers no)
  (pad "1" smd roundrect (at -0.48 0) (size 0.56 0.62) (layers "F.Cu" "F.Mask" "F.Paste") (roundrect_rratio 0.25) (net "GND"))
  (pad "2" smd roundrect (at 0.48 0) (size 0.56 0.62) (layers "F.Cu" "F.Mask" "F.Paste") (roundrect_rratio 0.25) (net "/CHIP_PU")))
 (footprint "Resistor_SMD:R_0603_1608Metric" (layer "F.Cu") (at 123.88 109.32)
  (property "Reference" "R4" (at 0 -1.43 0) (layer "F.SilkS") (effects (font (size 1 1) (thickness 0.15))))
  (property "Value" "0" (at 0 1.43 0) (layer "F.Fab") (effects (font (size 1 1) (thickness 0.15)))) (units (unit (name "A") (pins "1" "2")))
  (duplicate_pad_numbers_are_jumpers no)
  (pad "1" smd roundrect (at -0.825 0) (size 0.8 0.95) (layers "F.Cu" "F.Mask" "F.Paste") (roundrect_rratio 0.25) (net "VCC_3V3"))
  (pad "2" smd roundrect (at 0.825 0) (size 0.8 0.95) (layers "F.Cu" "F.Mask" "F.Paste") (roundrect_rratio 0.25) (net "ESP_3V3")))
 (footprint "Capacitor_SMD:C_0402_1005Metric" (layer "F.Cu") (at 148.52 108.5)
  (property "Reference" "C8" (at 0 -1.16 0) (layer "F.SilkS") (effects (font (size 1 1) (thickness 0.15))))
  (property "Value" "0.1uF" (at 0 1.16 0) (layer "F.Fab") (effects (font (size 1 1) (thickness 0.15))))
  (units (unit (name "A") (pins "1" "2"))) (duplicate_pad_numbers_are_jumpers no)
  (pad "1" smd roundrect (at -0.48 0) (size 0.56 0.62) (layers "F.Cu" "F.Mask" "F.Paste") (roundrect_rratio 0.25) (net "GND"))
  (pad "2" smd roundrect (at 0.48 0) (size 0.56 0.62) (layers "F.Cu" "F.Mask" "F.Paste") (roundrect_rratio 0.25) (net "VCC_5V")))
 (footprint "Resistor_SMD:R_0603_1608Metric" (layer "F.Cu") (at 123.88 114.34)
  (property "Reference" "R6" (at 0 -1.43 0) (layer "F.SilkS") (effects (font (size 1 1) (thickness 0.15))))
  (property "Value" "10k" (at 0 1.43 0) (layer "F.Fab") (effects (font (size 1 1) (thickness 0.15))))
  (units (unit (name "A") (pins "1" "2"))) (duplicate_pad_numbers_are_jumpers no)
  (pad "1" smd roundrect (at -0.825 0) (size 0.8 0.95) (layers "F.Cu" "F.Mask" "F.Paste") (roundrect_rratio 0.25) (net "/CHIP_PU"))
  (pad "2" smd roundrect (at 0.825 0) (size 0.8 0.95) (layers "F.Cu" "F.Mask" "F.Paste") (roundrect_rratio 0.25) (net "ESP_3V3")))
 (gr_rect (start 150 50) (end 171 122) (stroke (width 0.2) (type solid)) (fill no) (layer "Edge.Cuts"))
 (segment (start 153.52 72.88) (end 152 74.4) (width 0.2) (layer "F.Cu") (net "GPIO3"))
 (segment (start 153.52 68.78) (end 153.52 72.88) (width 0.2) (layer "F.Cu") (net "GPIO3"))
 (segment (start 153.232843 73.732843) (end 153.232843 75.707157) (width 0.2) (layer "F.Cu") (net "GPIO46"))
 (segment (start 153.92 73.045686) (end 153.232843 73.732843) (width 0.2) (layer "F.Cu") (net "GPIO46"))
 (segment (start 154.79 68.78) (end 154.79 69.63) (width 0.2) (layer "F.Cu") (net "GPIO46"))
 (segment (start 154.79 69.63) (end 153.92 70.5) (width 0.2) (layer "F.Cu") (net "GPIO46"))
 (segment (start 153.92 70.5) (end 153.92 73.045686) (width 0.2) (layer "F.Cu") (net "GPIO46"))
 (segment (start 153.232843 75.707157) (end 152 76.94) (width 0.2) (layer "F.Cu") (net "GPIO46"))
 (segment (start 156.06 69.73) (end 155.79 70) (width 0.2) (layer "F.Cu") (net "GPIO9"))
 (segment (start 153.398528 78.081472) (end 152 79.48) (width 0.2) (layer "F.Cu") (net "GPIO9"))
 (segment (start 154.32 70.68) (end 154.32 73.211372) (width 0.2) (layer "F.Cu") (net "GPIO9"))
 (segment (start 153.632843 73.898529) (end 153.632843 75.872843) (width 0.2) (layer "F.Cu") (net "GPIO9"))
 (segment (start 155.79 70) (end 155 70) (width 0.2) (layer "F.Cu") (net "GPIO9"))
 (segment (start 154.32 73.211372) (end 153.632843 73.898529) (width 0.2) (layer "F.Cu") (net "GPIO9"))
 (segment (start 155 70) (end 154.32 70.68) (width 0.2) (layer "F.Cu") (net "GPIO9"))
 (segment (start 153.632843 75.872843) (end 153.398528 76.107157) (width 0.2) (layer "F.Cu") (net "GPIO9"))
 (segment (start 156.06 68.78) (end 156.06 69.73) (width 0.2) (layer "F.Cu") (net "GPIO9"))
 (segment (start 153.398528 76.107157) (end 153.398528 78.081472) (width 0.2) (layer "F.Cu") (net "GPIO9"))
 (segment (start 154.032843 74.064215) (end 154.032842 76.265686) (width 0.2) (layer "F.Cu") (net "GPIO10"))
 (segment (start 153.564213 80.455787) (end 152 82.02) (width 0.2) (layer "F.Cu") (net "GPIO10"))
 (segment (start 156 70.5) (end 155.065686 70.5) (width 0.2) (layer "F.Cu") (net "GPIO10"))
 (segment (start 153.798528 76.5) (end 153.798528 78.247158) (width 0.2) (layer "F.Cu") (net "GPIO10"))
 (segment (start 155.065686 70.5) (end 154.72 70.845686) (width 0.2) (layer "F.Cu") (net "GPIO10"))
 (segment (start 153.798528 78.247158) (end 153.564213 78.481472) (width 0.2) (layer "F.Cu") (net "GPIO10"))
 (segment (start 153.564213 78.481472) (end 153.564213 80.455787) (width 0.2) (layer "F.Cu") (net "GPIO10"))
 (segment (start 157.33 68.78) (end 157.33 69.17) (width 0.2) (layer "F.Cu") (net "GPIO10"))
 (segment (start 154.032842 76.265686) (end 153.798528 76.5) (width 0.2) (layer "F.Cu") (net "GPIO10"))
 (segment (start 157.33 69.17) (end 156 70.5) (width 0.2) (layer "F.Cu") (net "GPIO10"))
 (segment (start 154.72 73.377057) (end 154.032843 74.064215) (width 0.2) (layer "F.Cu") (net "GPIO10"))
 (segment (start 154.72 70.845686) (end 154.72 73.377057) (width 0.2) (layer "F.Cu") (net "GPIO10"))
 (segment (start 158.6 69.73) (end 158.297157 70.032843) (width 0.2) (layer "F.Cu") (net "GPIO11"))
 (segment (start 154.198527 78.765686) (end 153.964213 79) (width 0.2) (layer "F.Cu") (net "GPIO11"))
 (segment (start 154.885685 73.777057) (end 154.432843 74.229901) (width 0.2) (layer "F.Cu") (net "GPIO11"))
 (segment (start 155.12 73.542743) (end 154.885685 73.777057) (width 0.2) (layer "F.Cu") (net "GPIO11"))
 (segment (start 154.198528 76.665686) (end 154.198527 78.765686) (width 0.2) (layer "F.Cu") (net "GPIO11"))
 (segment (start 156.065685 71) (end 155.5 71) (width 0.2) (layer "F.Cu") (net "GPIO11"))
 (segment (start 157.032843 70.032843) (end 156.065685 71) (width 0.2) (layer "F.Cu") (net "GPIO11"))
 (segment (start 153.729898 82.830102) (end 152 84.56) (width 0.2) (layer "F.Cu") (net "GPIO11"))
 (segment (start 158.6 68.78) (end 158.6 69.73) (width 0.2) (layer "F.Cu") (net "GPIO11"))
 (segment (start 153.964213 80.621473) (end 153.729898 80.855787) (width 0.2) (layer "F.Cu") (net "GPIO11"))
 (segment (start 153.729898 80.855787) (end 153.729898 82.830102) (width 0.2) (layer "F.Cu") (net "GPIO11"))
 (segment (start 154.432842 76.431372) (end 154.198528 76.665686) (width 0.2) (layer "F.Cu") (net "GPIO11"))
 (segment (start 158.297157 70.032843) (end 157.032843 70.032843) (width 0.2) (layer "F.Cu") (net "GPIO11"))
 (segment (start 155.5 71) (end 155.12 71.38) (width 0.2) (layer "F.Cu") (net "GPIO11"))
 (segment (start 153.964213 79) (end 153.964213 80.621473) (width 0.2) (layer "F.Cu") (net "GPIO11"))
 (segment (start 155.12 71.38) (end 155.12 73.542743) (width 0.2) (layer "F.Cu") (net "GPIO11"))
 (segment (start 154.432843 74.229901) (end 154.432842 76.431372) (width 0.2) (layer "F.Cu") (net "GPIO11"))
 (segment (start 154.598527 78.931372) (end 154.364212 79.165686) (width 0.2) (layer "F.Cu") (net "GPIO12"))
 (segment (start 154.129898 83.370102) (end 153.5 84) (width 0.2) (layer "F.Cu") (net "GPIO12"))
 (segment (start 154.129898 81.5) (end 154.129898 83.370102) (width 0.2) (layer "F.Cu") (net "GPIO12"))
 (segment (start 154.364212 81.265686) (end 154.129898 81.5) (width 0.2) (layer "F.Cu") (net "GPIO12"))
 (segment (start 155.519999 73.812844) (end 154.832843 74.5) (width 0.2) (layer "F.Cu") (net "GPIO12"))
 (segment (start 153.5 85.6) (end 152 87.1) (width 0.2) (layer "F.Cu") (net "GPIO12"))
 (segment (start 154.598528 77) (end 154.598527 78.931372) (width 0.2) (layer "F.Cu") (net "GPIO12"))
 (segment (start 157.131371 70.5) (end 155.52 72.111371) (width 0.2) (layer "F.Cu") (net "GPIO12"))
 (segment (start 159.1 70.5) (end 157.131371 70.5) (width 0.2) (layer "F.Cu") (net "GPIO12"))
 (segment (start 159.87 68.78) (end 159.87 69.73) (width 0.2) (layer "F.Cu") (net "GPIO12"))
 (segment (start 159.87 69.73) (end 159.1 70.5) (width 0.2) (layer "F.Cu") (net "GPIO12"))
 (segment (start 155.52 72.111371) (end 155.519999 73.812844) (width 0.2) (layer "F.Cu") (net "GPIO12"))
 (segment (start 153.5 84) (end 153.5 85.6) (width 0.2) (layer "F.Cu") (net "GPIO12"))
 (segment (start 154.364212 79.165686) (end 154.364212 81.265686) (width 0.2) (layer "F.Cu") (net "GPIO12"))
 (segment (start 154.832843 74.5) (end 154.832842 76.765686) (width 0.2) (layer "F.Cu") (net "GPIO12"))
 (segment (start 154.832842 76.765686) (end 154.598528 77) (width 0.2) (layer "F.Cu") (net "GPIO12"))
 (segment (start 160.83 105.1) (end 158.03 102.3) (width 0.2) (layer "F.Cu") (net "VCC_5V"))
 (segment (start 161 105.1) (end 160.83 105.1) (width 0.2) (layer "F.Cu") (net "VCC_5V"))
 (segment (start 158.1 115.507544) (end 158.1 116.242239) (width 0.2) (layer "F.Cu") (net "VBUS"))
 (segment (start 163.039848 115.367696) (end 162.9 115.507544) (width 0.2) (layer "F.Cu") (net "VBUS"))
 (segment (start 162.9 116.242239) (end 162.284695 116.857544) (width 0.2) (layer "F.Cu") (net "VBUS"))
 (segment (start 158.7 116.857544) (end 158.715305 116.857544) (width 0.2) (layer "F.Cu") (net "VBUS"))
 (segment (start 163.039848 114.708876) (end 163.039848 115.367696) (width 0.2) (layer "F.Cu") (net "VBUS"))
 (segment (start 164 109.5) (end 164 113.748724) (width 0.2) (layer "F.Cu") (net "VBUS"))
 (segment (start 160.999999 110.225001) (end 161 107.9) (width 0.2) (layer "F.Cu") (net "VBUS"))
 (segment (start 162.7 115.707544) (end 162.9 115.507544) (width 0.2) (layer "F.Cu") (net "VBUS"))
 (segment (start 158.715305 116.857544) (end 162.284695 116.857544) (width 0.2) (layer "F.Cu") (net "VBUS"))
 (segment (start 158.1 116.242239) (end 158.715305 116.857544) (width 0.2) (layer "F.Cu") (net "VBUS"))
 (segment (start 162.4 107.9) (end 164 109.5) (width 0.2) (layer "F.Cu") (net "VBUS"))
 (segment (start 158.1 115.507544) (end 158.3 115.707544) (width 0.2) (layer "F.Cu") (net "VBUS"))
 (segment (start 162.9 115.507544) (end 162.9 116.242239) (width 0.2) (layer "F.Cu") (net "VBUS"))
 (segment (start 163.039848 114.708876) (end 164 113.748724) (width 0.2) (layer "F.Cu") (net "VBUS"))
 (segment (start 161 107.9) (end 162.4 107.9) (width 0.2) (layer "F.Cu") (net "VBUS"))
 (segment (start 160.7 114.557544) (end 159.8 114.557544) (width 0.2) (layer "F.Cu") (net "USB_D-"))
 (segment (start 160.75 115.507544) (end 160.75 114.607544) (width 0.2) (layer "F.Cu") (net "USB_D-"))
 (segment (start 159.8 114.557544) (end 159.75 114.607544) (width 0.2) (layer "F.Cu") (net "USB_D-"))
 (segment (start 160.75 115.507544) (end 160.75 114.532543) (width 0.2) (layer "F.Cu") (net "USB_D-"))
 (segment (start 159.75 114.607544) (end 159.75 115.507544) (width 0.2) (layer "F.Cu") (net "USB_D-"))
 (segment (start 160.659449 113.462499) (end 160.400001 113.203051) (width 0.2) (layer "F.Cu") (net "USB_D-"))
 (segment (start 160.400001 112.849999) (end 160.050001 112.499999) (width 0.2) (layer "F.Cu") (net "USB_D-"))
 (segment (start 160.775 113.462499) (end 160.659449 113.462499) (width 0.2) (layer "F.Cu") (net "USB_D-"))
 (segment (start 160.775 114.507543) (end 160.775 113.462499) (width 0.2) (layer "F.Cu") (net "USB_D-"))
 (segment (start 160.400001 113.203051) (end 160.400001 112.849999) (width 0.2) (layer "F.Cu") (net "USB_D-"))
 (segment (start 160.75 114.607544) (end 160.7 114.557544) (width 0.2) (layer "F.Cu") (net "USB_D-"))
 (segment (start 160.75 114.532543) (end 160.775 114.507543) (width 0.2) (layer "F.Cu") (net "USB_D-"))
 (segment (start 161.225003 113.687496) (end 161.225003 113.462499) (width 0.2) (layer "F.Cu") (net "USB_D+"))
 (segment (start 161.2 116.457544) (end 160.3 116.457544) (width 0.2) (layer "F.Cu") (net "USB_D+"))
 (segment (start 161.25 115.507544) (end 161.25 114.532543) (width 0.2) (layer "F.Cu") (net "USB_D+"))
 (segment (start 161.600001 112.850001) (end 161.950001 112.500001) (width 0.2) (layer "F.Cu") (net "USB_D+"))
 (segment (start 160.25 116.407544) (end 160.25 115.507544) (width 0.2) (layer "F.Cu") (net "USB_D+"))
 (segment (start 161.25 114.532543) (end 161.225 114.507543) (width 0.2) (layer "F.Cu") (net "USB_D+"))
 (segment (start 161.225 113.687499) (end 161.225003 113.687496) (width 0.2) (layer "F.Cu") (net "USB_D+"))
 (segment (start 161.600001 113.203051) (end 161.600001 112.850001) (width 0.2) (layer "F.Cu") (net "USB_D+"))
 (segment (start 161.25 116.407544) (end 161.2 116.457544) (width 0.2) (layer "F.Cu") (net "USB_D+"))
 (segment (start 160.3 116.457544) (end 160.25 116.407544) (width 0.2) (layer "F.Cu") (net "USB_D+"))
 (segment (start 161.25 115.507544) (end 161.25 116.407544) (width 0.2) (layer "F.Cu") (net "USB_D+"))
 (segment (start 161.225 114.507543) (end 161.225 113.687499) (width 0.2) (layer "F.Cu") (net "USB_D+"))
 (segment (start 161.225003 113.462499) (end 161.340553 113.462499) (width 0.2) (layer "F.Cu") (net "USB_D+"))
 (segment (start 161.340553 113.462499) (end 161.600001 113.203051) (width 0.2) (layer "F.Cu") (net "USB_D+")))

